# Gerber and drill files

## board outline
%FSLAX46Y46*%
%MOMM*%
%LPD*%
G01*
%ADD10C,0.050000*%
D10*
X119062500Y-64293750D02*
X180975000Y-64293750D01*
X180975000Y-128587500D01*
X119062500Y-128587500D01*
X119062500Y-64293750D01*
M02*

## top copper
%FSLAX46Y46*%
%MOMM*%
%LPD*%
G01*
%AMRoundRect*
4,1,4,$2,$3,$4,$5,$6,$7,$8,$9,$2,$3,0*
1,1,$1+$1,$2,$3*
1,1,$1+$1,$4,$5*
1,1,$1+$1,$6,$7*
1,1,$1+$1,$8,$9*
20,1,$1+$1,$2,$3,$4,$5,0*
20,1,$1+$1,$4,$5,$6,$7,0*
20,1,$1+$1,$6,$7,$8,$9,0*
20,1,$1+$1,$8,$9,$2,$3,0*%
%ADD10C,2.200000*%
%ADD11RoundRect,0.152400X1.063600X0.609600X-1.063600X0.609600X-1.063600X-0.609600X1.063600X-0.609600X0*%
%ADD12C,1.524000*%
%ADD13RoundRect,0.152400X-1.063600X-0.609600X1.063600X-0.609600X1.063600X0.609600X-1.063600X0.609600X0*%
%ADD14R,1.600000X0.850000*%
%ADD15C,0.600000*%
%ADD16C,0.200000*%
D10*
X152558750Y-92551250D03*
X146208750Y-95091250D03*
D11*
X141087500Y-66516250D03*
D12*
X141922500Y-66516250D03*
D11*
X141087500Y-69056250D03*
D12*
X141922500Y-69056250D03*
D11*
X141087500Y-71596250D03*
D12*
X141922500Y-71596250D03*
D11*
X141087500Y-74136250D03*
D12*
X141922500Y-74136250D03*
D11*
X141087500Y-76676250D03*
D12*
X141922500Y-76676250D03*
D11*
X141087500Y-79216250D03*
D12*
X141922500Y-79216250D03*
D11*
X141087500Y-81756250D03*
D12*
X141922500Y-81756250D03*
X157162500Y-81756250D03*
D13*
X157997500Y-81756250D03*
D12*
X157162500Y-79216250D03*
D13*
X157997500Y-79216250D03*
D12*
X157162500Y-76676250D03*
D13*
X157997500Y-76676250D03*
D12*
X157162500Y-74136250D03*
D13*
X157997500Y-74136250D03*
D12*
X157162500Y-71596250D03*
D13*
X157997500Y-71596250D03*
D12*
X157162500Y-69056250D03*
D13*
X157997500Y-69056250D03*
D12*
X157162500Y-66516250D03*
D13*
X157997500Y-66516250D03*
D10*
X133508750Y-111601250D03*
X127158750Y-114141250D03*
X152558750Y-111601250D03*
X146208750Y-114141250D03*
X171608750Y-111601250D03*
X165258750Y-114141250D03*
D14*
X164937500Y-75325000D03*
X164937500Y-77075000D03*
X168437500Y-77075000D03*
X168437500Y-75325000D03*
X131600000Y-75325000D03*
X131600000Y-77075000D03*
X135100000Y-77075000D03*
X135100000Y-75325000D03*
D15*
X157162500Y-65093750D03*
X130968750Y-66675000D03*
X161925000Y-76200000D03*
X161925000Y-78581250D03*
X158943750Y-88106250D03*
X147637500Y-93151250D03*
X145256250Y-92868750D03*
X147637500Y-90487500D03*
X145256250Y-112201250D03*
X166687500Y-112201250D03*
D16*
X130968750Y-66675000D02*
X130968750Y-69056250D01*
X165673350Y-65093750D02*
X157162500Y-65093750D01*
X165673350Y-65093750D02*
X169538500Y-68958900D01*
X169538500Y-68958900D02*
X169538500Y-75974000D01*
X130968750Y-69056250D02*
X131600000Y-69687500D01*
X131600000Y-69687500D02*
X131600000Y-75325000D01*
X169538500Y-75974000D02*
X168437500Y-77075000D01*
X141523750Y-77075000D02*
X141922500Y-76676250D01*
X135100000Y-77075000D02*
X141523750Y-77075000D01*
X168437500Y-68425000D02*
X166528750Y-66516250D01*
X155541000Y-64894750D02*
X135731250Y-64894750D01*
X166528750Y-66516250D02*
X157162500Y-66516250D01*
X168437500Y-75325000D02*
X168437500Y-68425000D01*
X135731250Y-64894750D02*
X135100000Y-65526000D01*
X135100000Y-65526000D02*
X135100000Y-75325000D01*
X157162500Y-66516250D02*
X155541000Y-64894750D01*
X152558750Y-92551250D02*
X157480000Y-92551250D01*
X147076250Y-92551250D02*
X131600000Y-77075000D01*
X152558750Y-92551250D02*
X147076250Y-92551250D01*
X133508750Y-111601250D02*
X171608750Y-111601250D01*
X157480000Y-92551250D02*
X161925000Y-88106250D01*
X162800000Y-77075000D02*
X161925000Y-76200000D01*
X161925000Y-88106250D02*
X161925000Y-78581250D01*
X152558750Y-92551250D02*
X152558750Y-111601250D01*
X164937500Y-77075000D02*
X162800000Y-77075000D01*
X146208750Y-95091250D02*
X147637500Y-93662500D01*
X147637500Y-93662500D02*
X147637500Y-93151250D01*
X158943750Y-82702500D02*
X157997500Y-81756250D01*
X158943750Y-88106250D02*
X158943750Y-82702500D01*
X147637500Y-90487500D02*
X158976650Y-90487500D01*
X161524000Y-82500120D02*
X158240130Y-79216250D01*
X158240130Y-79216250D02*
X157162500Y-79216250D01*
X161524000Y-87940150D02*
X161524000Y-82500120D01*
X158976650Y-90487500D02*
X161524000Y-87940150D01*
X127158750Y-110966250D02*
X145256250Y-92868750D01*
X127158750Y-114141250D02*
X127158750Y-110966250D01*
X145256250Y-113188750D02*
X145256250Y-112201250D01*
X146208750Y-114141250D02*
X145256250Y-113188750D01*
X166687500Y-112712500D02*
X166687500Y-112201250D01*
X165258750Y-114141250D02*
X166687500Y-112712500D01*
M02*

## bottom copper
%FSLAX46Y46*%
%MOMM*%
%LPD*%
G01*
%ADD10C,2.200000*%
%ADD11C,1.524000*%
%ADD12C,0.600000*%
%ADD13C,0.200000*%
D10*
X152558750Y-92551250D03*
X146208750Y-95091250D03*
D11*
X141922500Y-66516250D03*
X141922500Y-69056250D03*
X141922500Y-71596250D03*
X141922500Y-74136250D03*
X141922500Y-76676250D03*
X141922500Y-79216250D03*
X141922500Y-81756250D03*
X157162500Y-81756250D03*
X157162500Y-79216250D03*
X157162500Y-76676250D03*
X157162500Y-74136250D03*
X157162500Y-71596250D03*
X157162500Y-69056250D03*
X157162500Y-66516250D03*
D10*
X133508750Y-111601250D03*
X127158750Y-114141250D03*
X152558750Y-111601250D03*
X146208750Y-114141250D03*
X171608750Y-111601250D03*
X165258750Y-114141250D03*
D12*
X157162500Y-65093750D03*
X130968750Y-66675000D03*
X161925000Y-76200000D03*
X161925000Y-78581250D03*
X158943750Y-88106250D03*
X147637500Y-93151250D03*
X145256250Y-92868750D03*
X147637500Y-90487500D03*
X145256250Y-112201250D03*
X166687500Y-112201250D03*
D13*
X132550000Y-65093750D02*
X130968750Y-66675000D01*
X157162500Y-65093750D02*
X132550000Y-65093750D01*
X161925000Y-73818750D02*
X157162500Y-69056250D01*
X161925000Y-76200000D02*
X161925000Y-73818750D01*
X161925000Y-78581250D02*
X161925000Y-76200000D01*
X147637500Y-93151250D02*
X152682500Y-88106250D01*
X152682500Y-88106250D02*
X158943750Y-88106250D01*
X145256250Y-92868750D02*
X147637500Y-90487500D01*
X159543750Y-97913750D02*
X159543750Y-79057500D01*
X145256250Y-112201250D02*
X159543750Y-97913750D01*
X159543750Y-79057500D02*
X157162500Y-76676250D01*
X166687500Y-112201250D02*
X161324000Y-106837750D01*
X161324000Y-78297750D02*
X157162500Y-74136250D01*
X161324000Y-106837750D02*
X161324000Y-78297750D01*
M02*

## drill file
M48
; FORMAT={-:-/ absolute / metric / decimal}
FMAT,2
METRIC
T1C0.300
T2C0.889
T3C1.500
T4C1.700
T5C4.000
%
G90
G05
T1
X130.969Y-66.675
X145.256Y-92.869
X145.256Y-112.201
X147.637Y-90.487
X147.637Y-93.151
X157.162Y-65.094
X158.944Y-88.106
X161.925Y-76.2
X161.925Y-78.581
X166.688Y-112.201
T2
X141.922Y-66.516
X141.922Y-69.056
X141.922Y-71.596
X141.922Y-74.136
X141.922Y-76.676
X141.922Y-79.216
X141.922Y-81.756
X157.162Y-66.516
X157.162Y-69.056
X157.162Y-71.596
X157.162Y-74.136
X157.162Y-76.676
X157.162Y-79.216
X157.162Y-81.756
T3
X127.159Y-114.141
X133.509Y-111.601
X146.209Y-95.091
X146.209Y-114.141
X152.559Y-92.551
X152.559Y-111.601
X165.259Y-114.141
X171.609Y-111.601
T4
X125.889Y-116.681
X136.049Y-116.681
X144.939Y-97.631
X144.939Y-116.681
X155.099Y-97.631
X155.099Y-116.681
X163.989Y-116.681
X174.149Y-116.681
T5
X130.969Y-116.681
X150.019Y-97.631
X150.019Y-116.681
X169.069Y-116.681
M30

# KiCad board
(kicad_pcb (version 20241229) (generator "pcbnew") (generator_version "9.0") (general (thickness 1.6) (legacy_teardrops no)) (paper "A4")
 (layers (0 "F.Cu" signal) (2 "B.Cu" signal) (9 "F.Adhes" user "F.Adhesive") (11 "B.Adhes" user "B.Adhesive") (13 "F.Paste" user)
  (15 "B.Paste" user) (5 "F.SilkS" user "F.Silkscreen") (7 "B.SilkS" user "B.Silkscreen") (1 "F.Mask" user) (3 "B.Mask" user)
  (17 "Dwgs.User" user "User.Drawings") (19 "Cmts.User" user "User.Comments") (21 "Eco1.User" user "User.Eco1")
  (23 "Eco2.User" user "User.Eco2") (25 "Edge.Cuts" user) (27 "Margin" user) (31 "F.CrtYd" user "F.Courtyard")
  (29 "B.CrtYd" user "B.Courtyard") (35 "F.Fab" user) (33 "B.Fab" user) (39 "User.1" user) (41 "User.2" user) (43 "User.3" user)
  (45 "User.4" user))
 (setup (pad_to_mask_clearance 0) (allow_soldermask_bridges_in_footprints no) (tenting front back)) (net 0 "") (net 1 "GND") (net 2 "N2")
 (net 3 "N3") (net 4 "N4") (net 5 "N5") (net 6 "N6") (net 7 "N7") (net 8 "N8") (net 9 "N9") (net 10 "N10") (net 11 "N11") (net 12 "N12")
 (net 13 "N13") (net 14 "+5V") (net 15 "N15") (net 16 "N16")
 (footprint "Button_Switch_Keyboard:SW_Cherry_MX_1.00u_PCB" (layer "F.Cu") (at 152.55875 92.55125)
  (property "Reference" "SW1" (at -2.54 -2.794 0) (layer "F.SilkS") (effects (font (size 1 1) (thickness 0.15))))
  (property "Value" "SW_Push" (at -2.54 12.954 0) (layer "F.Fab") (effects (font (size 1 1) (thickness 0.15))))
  (pad "" np_thru_hole circle (at -7.62 5.08) (size 1.7 1.7) (drill 1.7) (layers "*.Cu" "*.Mask"))
  (pad "" np_thru_hole circle (at -2.54 5.08) (size 4 4) (drill 4) (layers "*.Cu" "*.Mask"))
  (pad "" np_thru_hole circle (at 2.54 5.08) (size 1.7 1.7) (drill 1.7) (layers "*.Cu" "*.Mask"))
  (pad "1" thru_hole circle (at 0 0) (size 2.2 2.2) (drill 1.5) (layers "*.Cu" "*.Mask") (remove_unused_layers no) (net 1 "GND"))
  (pad "2" thru_hole circle (at -6.35 2.54) (size 2.2 2.2) (drill 1.5) (layers "*.Cu" "*.Mask") (remove_unused_layers no) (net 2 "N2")))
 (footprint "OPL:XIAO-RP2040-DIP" (layer "F.Cu") (at 149.5425 74.13625)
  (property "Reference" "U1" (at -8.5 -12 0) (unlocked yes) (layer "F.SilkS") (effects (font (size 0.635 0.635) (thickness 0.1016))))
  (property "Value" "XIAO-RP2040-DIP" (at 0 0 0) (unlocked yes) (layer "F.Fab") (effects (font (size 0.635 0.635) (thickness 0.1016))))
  (pad "1" smd roundrect (at -8.455 -7.62 180) (size 2.432 1.524) (layers "F.Cu" "F.Mask") (roundrect_rratio 0.1) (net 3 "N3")
   (thermal_bridge_angle 45))
  (pad "1" thru_hole circle (at -7.62 -7.62 180) (size 1.524 1.524) (drill 0.889) (layers "*.Cu" "*.Mask") (remove_unused_layers no)
   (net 3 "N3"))
  (pad "2" smd roundrect (at -8.455 -5.08 180) (size 2.432 1.524) (layers "F.Cu" "F.Mask") (roundrect_rratio 0.1) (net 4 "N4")
   (thermal_bridge_angle 45))
  (pad "2" thru_hole circle (at -7.62 -5.08 180) (size 1.524 1.524) (drill 0.889) (layers "*.Cu" "*.Mask") (remove_unused_layers no)
   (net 4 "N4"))
  (pad "3" smd roundrect (at -8.455 -2.54 180) (size 2.432 1.524) (layers "F.Cu" "F.Mask") (roundrect_rratio 0.1) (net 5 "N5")
   (thermal_bridge_angle 45))
  (pad "3" thru_hole circle (at -7.62 -2.54 180) (size 1.524 1.524) (drill 0.889) (layers "*.Cu" "*.Mask") (remove_unused_layers no)
   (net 5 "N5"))
  (pad "4" smd roundrect (at -8.455 0 180) (size 2.432 1.524) (layers "F.Cu" "F.Mask") (roundrect_rratio 0.1) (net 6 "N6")
   (thermal_bridge_angle 45))
  (pad "4" thru_hole circle (at -7.62 0 180) (size 1.524 1.524) (drill 0.889) (layers "*.Cu" "*.Mask") (remove_unused_layers no)
   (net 6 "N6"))
  (pad "5" smd roundrect (at -8.455 2.54 180) (size 2.432 1.524) (layers "F.Cu" "F.Mask") (roundrect_rratio 0.1) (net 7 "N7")
   (thermal_bridge_angle 45))
  (pad "5" thru_hole circle (at -7.62 2.54 180) (size 1.524 1.524) (drill 0.889) (layers "*.Cu" "*.Mask") (remove_unused_layers no)
   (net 7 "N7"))
  (pad "6" smd roundrect (at -8.455 5.08 180) (size 2.432 1.524) (layers "F.Cu" "F.Mask") (roundrect_rratio 0.1) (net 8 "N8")
   (thermal_bridge_angle 45))
  (pad "6" thru_hole circle (at -7.62 5.08 180) (size 1.524 1.524) (drill 0.889) (layers "*.Cu" "*.Mask") (remove_unused_layers no)
   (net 8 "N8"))
  (pad "7" smd roundrect (at -8.455 7.62 180) (size 2.432 1.524) (layers "F.Cu" "F.Mask") (roundrect_rratio 0.1) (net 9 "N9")
   (thermal_bridge_angle 45))
  (pad "7" thru_hole circle (at -7.62 7.62 180) (size 1.524 1.524) (drill 0.889) (layers "*.Cu" "*.Mask") (remove_unused_layers no)
   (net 9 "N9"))
  (pad "8" thru_hole circle (at 7.62 7.62) (size 1.524 1.524) (drill 0.889) (layers "*.Cu" "*.Mask") (remove_unused_layers no) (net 2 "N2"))
  (pad "8" smd roundrect (at 8.455 7.62) (size 2.432 1.524) (layers "F.Cu" "F.Mask") (roundrect_rratio 0.1) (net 2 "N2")
   (thermal_bridge_angle 45))
  (pad "9" thru_hole circle (at 7.62 5.08) (size 1.524 1.524) (drill 0.889) (layers "*.Cu" "*.Mask") (remove_unused_layers no)
   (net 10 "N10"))
  (pad "9" smd roundrect (at 8.455 5.08) (size 2.432 1.524) (layers "F.Cu" "F.Mask") (roundrect_rratio 0.1) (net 10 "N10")
   (thermal_bridge_angle 45))
  (pad "10" thru_hole circle (at 7.62 2.54) (size 1.524 1.524) (drill 0.889) (layers "*.Cu" "*.Mask") (remove_unused_layers no)
   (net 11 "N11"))
  (pad "10" smd roundrect (at 8.455 2.54) (size 2.432 1.524) (layers "F.Cu" "F.Mask") (roundrect_rratio 0.1) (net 11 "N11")
   (thermal_bridge_angle 45))
  (pad "11" thru_hole circle (at 7.62 0) (size 1.524 1.524) (drill 0.889) (layers "*.Cu" "*.Mask") (remove_unused_layers no) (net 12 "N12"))
  (pad "11" smd roundrect (at 8.455 0) (size 2.432 1.524) (layers "F.Cu" "F.Mask") (roundrect_rratio 0.1) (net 12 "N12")
   (thermal_bridge_angle 45))
  (pad "12" thru_hole circle (at 7.62 -2.54) (size 1.524 1.524) (drill 0.889) (layers "*.Cu" "*.Mask") (remove_unused_layers no)
   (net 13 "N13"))
  (pad "12" smd roundrect (at 8.455 -2.54) (size 2.432 1.524) (layers "F.Cu" "F.Mask") (roundrect_rratio 0.1) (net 13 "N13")
   (thermal_bridge_angle 45))
  (pad "13" thru_hole circle (at 7.62 -5.08) (size 1.524 1.524) (drill 0.889) (layers "*.Cu" "*.Mask") (remove_unused_layers no)
   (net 1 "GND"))
  (pad "13" smd roundrect (at 8.455 -5.08) (size 2.432 1.524) (layers "F.Cu" "F.Mask") (roundrect_rratio 0.1) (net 1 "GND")
   (thermal_bridge_angle 45))
  (pad "14" thru_hole circle (at 7.62 -7.62) (size 1.524 1.524) (drill 0.889) (layers "*.Cu" "*.Mask") (remove_unused_layers no)
   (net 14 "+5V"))
  (pad "14" smd roundrect (at 8.455 -7.62) (size 2.432 1.524) (layers "F.Cu" "F.Mask") (roundrect_rratio 0.1) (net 14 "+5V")
   (thermal_bridge_angle 45)))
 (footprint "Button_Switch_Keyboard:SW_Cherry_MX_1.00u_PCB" (layer "F.Cu") (at 133.50875 111.60125)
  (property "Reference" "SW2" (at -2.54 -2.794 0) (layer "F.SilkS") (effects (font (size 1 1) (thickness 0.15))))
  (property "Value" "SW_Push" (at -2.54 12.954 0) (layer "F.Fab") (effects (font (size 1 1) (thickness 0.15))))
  (pad "" np_thru_hole circle (at -7.62 5.08) (size 1.7 1.7) (drill 1.7) (layers "*.Cu" "*.Mask"))
  (pad "" np_thru_hole circle (at -2.54 5.08) (size 4 4) (drill 4) (layers "*.Cu" "*.Mask"))
  (pad "" np_thru_hole circle (at 2.54 5.08) (size 1.7 1.7) (drill 1.7) (layers "*.Cu" "*.Mask"))
  (pad "1" thru_hole circle (at 0 0) (size 2.2 2.2) (drill 1.5) (layers "*.Cu" "*.Mask") (remove_unused_layers no) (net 1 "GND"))
  (pad "2" thru_hole circle (at -6.35 2.54) (size 2.2 2.2) (drill 1.5) (layers "*.Cu" "*.Mask") (remove_unused_layers no) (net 10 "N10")))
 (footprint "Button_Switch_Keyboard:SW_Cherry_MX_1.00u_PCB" (layer "F.Cu") (at 152.55875 111.60125)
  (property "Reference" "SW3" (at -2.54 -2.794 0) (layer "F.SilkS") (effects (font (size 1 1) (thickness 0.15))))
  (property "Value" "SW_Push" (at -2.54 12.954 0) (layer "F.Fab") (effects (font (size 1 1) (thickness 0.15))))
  (pad "" np_thru_hole circle (at -7.62 5.08) (size 1.7 1.7) (drill 1.7) (layers "*.Cu" "*.Mask"))
  (pad "" np_thru_hole circle (at -2.54 5.08) (size 4 4) (drill 4) (layers "*.Cu" "*.Mask"))
  (pad "" np_thru_hole circle (at 2.54 5.08) (size 1.7 1.7) (drill 1.7) (layers "*.Cu" "*.Mask"))
  (pad "1" thru_hole circle (at 0 0) (size 2.2 2.2) (drill 1.5) (layers "*.Cu" "*.Mask") (remove_unused_layers no) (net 1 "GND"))
  (pad "2" thru_hole circle (at -6.35 2.54) (size 2.2 2.2) (drill 1.5) (layers "*.Cu" "*.Mask") (remove_unused_layers no) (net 11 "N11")))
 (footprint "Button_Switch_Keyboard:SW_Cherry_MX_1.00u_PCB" (layer "F.Cu") (at 171.60875 111.60125)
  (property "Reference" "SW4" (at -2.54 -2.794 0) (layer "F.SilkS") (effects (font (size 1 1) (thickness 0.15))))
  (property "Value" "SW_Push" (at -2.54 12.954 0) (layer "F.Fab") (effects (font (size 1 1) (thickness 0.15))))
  (pad "" np_thru_hole circle (at -7.62 5.08) (size 1.7 1.7) (drill 1.7) (layers "*.Cu" "*.Mask"))
  (pad "" np_thru_hole circle (at -2.54 5.08) (size 4 4) (drill 4) (layers "*.Cu" "*.Mask"))
  (pad "" np_thru_hole circle (at 2.54 5.08) (size 1.7 1.7) (drill 1.7) (layers "*.Cu" "*.Mask"))
  (pad "1" thru_hole circle (at 0 0) (size 2.2 2.2) (drill 1.5) (layers "*.Cu" "*.Mask") (remove_unused_layers no) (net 1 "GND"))
  (pad "2" thru_hole circle (at -6.35 2.54) (size 2.2 2.2) (drill 1.5) (layers "*.Cu" "*.Mask") (remove_unused_layers no) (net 12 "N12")))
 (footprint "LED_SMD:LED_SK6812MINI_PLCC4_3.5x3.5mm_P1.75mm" (layer "F.Cu") (at 166.6875 76.2)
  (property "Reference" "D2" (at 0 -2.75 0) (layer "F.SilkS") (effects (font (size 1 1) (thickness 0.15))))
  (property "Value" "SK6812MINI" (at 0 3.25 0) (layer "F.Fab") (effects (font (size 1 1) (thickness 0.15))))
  (pad "1" smd rect (at -1.75 -0.875) (size 1.6 0.85) (layers "F.Cu" "F.Mask" "F.Paste") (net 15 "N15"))
  (pad "2" smd rect (at -1.75 0.875) (size 1.6 0.85) (layers "F.Cu" "F.Mask" "F.Paste") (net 1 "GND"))
  (pad "3" smd rect (at 1.75 0.875) (size 1.6 0.85) (layers "F.Cu" "F.Mask" "F.Paste") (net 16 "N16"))
  (pad "4" smd rect (at 1.75 -0.875) (size 1.6 0.85) (layers "F.Cu" "F.Mask" "F.Paste") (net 14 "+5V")))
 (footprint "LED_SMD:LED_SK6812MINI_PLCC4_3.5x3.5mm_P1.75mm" (layer "F.Cu") (at 133.35 76.2)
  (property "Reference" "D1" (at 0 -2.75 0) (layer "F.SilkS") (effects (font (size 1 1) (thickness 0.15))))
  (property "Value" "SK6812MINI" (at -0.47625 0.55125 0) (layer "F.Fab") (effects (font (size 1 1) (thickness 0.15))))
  (pad "1" smd rect (at -1.75 -0.875) (size 1.6 0.85) (layers "F.Cu" "F.Mask" "F.Paste") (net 16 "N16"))
  (pad "2" smd rect (at -1.75 0.875) (size 1.6 0.85) (layers "F.Cu" "F.Mask" "F.Paste") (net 1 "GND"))
  (pad "3" smd rect (at 1.75 0.875) (size 1.6 0.85) (layers "F.Cu" "F.Mask" "F.Paste") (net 7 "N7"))
  (pad "4" smd rect (at 1.75 -0.875) (size 1.6 0.85) (layers "F.Cu" "F.Mask" "F.Paste") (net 14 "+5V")))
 (gr_rect (start 119.0625 64.29375) (end 180.975 128.5875) (stroke (width 0.05) (type default)) (fill no) (layer "Edge.Cuts"))
 (segment (start 130.96875 66.675) (end 130.96875 69.05625) (width 0.2) (layer "F.Cu") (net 16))
 (segment (start 165.67335 65.09375) (end 157.1625 65.09375) (width 0.2) (layer "F.Cu") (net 16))
 (segment (start 165.67335 65.09375) (end 169.5385 68.9589) (width 0.2) (layer "F.Cu") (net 16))
 (segment (start 169.5385 68.9589) (end 169.5385 75.974) (width 0.2) (layer "F.Cu") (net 16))
 (segment (start 130.96875 69.05625) (end 131.6 69.6875) (width 0.2) (layer "F.Cu") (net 16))
 (segment (start 131.6 69.6875) (end 131.6 75.325) (width 0.2) (layer "F.Cu") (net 16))
 (segment (start 169.5385 75.974) (end 168.4375 77.075) (width 0.2) (layer "F.Cu") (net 16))
 (via (at 157.1625 65.09375) (size 0.6) (drill 0.3) (layers "F.Cu" "B.Cu") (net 16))
 (via (at 130.96875 66.675) (size 0.6) (drill 0.3) (layers "F.Cu" "B.Cu") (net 16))
 (segment (start 132.55 65.09375) (end 130.96875 66.675) (width 0.2) (layer "B.Cu") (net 16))
 (segment (start 157.1625 65.09375) (end 132.55 65.09375) (width 0.2) (layer "B.Cu") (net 16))
 (segment (start 141.52375 77.075) (end 141.9225 76.67625) (width 0.2) (layer "F.Cu") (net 7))
 (segment (start 135.1 77.075) (end 141.52375 77.075) (width 0.2) (layer "F.Cu") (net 7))
 (segment (start 168.4375 68.425) (end 166.52875 66.51625) (width 0.2) (layer "F.Cu") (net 14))
 (segment (start 155.541 64.89475) (end 135.73125 64.89475) (width 0.2) (layer "F.Cu") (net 14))
 (segment (start 166.52875 66.51625) (end 157.1625 66.51625) (width 0.2) (layer "F.Cu") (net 14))
 (segment (start 168.4375 75.325) (end 168.4375 68.425) (width 0.2) (layer "F.Cu") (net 14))
 (segment (start 135.73125 64.89475) (end 135.1 65.526) (width 0.2) (layer "F.Cu") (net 14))
 (segment (start 135.1 65.526) (end 135.1 75.325) (width 0.2) (layer "F.Cu") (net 14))
 (segment (start 157.1625 66.51625) (end 155.541 64.89475) (width 0.2) (layer "F.Cu") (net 14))
 (segment (start 152.55875 92.55125) (end 157.48 92.55125) (width 0.2) (layer "F.Cu") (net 1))
 (segment (start 147.07625 92.55125) (end 131.6 77.075) (width 0.2) (layer "F.Cu") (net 1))
 (segment (start 152.55875 92.55125) (end 147.07625 92.55125) (width 0.2) (layer "F.Cu") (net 1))
 (segment (start 133.50875 111.60125) (end 171.60875 111.60125) (width 0.2) (layer "F.Cu") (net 1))
 (segment (start 157.48 92.55125) (end 161.925 88.10625) (width 0.2) (layer "F.Cu") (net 1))
 (segment (start 162.8 77.075) (end 161.925 76.2) (width 0.2) (layer "F.Cu") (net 1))
 (segment (start 161.925 88.10625) (end 161.925 78.58125) (width 0.2) (layer "F.Cu") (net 1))
 (segment (start 152.55875 92.55125) (end 152.55875 111.60125) (width 0.2) (layer "F.Cu") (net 1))
 (segment (start 164.9375 77.075) (end 162.8 77.075) (width 0.2) (layer "F.Cu") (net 1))
 (via (at 161.925 76.2) (size 0.6) (drill 0.3) (layers "F.Cu" "B.Cu") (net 1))
 (via (at 161.925 78.58125) (size 0.6) (drill 0.3) (layers "F.Cu" "B.Cu") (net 1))
 (segment (start 161.925 73.81875) (end 157.1625 69.05625) (width 0.2) (layer "B.Cu") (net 1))
 (segment (start 161.925 76.2) (end 161.925 73.81875) (width 0.2) (layer "B.Cu") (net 1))
 (segment (start 161.925 78.58125) (end 161.925 76.2) (width 0.2) (layer "B.Cu") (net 1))
 (segment (start 146.20875 95.09125) (end 147.6375 93.6625) (width 0.2) (layer "F.Cu") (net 2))
 (segment (start 147.6375 93.6625) (end 147.6375 93.15125) (width 0.2) (layer "F.Cu") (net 2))
 (segment (start 158.94375 82.7025) (end 157.9975 81.75625) (width 0.2) (layer "F.Cu") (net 2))
 (segment (start 158.94375 88.10625) (end 158.94375 82.7025) (width 0.2) (layer "F.Cu") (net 2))
 (via (at 158.94375 88.10625) (size 0.6) (drill 0.3) (layers "F.Cu" "B.Cu") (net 2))
 (via (at 147.6375 93.15125) (size 0.6) (drill 0.3) (layers "F.Cu" "B.Cu") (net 2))
 (segment (start 147.6375 93.15125) (end 152.6825 88.10625) (width 0.2) (layer "B.Cu") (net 2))
 (segment (start 152.6825 88.10625) (end 158.94375 88.10625) (width 0.2) (layer "B.Cu") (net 2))
 (segment (start 147.6375 90.4875) (end 158.97665 90.4875) (width 0.2) (layer "F.Cu") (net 10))
 (segment (start 161.524 82.50012) (end 158.24013 79.21625) (width 0.2) (layer "F.Cu") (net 10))
 (segment (start 158.24013 79.21625) (end 157.1625 79.21625) (width 0.2) (layer "F.Cu") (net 10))
 (segment (start 161.524 87.94015) (end 161.524 82.50012) (width 0.2) (layer "F.Cu") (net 10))
 (segment (start 158.97665 90.4875) (end 161.524 87.94015) (width 0.2) (layer "F.Cu") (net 10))
 (segment (start 127.15875 110.96625) (end 145.25625 92.86875) (width 0.2) (layer "F.Cu") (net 10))
 (segment (start 127.15875 114.14125) (end 127.15875 110.96625) (width 0.2) (layer "F.Cu") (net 10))
 (via (at 145.25625 92.86875) (size 0.6) (drill 0.3) (layers "F.Cu" "B.Cu") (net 10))
 (via (at 147.6375 90.4875) (size 0.6) (drill 0.3) (layers "F.Cu" "B.Cu") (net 10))
 (segment (start 145.25625 92.86875) (end 147.6375 90.4875) (width 0.2) (layer "B.Cu") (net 10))
 (segment (start 145.25625 113.18875) (end 145.25625 112.20125) (width 0.2) (layer "F.Cu") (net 11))
 (segment (start 146.20875 114.14125) (end 145.25625 113.18875) (width 0.2) (layer "F.Cu") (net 11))
 (via (at 145.25625 112.20125) (size 0.6) (drill 0.3) (layers "F.Cu" "B.Cu") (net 11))
 (segment (start 159.54375 97.91375) (end 159.54375 79.0575) (width 0.2) (layer "B.Cu") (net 11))
 (segment (start 145.25625 112.20125) (end 159.54375 97.91375) (width 0.2) (layer "B.Cu") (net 11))
 (segment (start 159.54375 79.0575) (end 157.1625 76.67625) (width 0.2) (layer "B.Cu") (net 11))
 (segment (start 166.6875 112.7125) (end 166.6875 112.20125) (width 0.2) (layer "F.Cu") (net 12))
 (segment (start 165.25875 114.14125) (end 166.6875 112.7125) (width 0.2) (layer "F.Cu") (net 12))
 (via (at 166.6875 112.20125) (size 0.6) (drill 0.3) (layers "F.Cu" "B.Cu") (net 12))
 (segment (start 166.6875 112.20125) (end 161.324 106.83775) (width 0.2) (layer "B.Cu") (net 12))
 (segment (start 161.324 78.29775) (end 157.1625 74.13625) (width 0.2) (layer "B.Cu") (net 12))
 (segment (start 161.324 106.83775) (end 161.324 78.29775) (width 0.2) (layer "B.Cu") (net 12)))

